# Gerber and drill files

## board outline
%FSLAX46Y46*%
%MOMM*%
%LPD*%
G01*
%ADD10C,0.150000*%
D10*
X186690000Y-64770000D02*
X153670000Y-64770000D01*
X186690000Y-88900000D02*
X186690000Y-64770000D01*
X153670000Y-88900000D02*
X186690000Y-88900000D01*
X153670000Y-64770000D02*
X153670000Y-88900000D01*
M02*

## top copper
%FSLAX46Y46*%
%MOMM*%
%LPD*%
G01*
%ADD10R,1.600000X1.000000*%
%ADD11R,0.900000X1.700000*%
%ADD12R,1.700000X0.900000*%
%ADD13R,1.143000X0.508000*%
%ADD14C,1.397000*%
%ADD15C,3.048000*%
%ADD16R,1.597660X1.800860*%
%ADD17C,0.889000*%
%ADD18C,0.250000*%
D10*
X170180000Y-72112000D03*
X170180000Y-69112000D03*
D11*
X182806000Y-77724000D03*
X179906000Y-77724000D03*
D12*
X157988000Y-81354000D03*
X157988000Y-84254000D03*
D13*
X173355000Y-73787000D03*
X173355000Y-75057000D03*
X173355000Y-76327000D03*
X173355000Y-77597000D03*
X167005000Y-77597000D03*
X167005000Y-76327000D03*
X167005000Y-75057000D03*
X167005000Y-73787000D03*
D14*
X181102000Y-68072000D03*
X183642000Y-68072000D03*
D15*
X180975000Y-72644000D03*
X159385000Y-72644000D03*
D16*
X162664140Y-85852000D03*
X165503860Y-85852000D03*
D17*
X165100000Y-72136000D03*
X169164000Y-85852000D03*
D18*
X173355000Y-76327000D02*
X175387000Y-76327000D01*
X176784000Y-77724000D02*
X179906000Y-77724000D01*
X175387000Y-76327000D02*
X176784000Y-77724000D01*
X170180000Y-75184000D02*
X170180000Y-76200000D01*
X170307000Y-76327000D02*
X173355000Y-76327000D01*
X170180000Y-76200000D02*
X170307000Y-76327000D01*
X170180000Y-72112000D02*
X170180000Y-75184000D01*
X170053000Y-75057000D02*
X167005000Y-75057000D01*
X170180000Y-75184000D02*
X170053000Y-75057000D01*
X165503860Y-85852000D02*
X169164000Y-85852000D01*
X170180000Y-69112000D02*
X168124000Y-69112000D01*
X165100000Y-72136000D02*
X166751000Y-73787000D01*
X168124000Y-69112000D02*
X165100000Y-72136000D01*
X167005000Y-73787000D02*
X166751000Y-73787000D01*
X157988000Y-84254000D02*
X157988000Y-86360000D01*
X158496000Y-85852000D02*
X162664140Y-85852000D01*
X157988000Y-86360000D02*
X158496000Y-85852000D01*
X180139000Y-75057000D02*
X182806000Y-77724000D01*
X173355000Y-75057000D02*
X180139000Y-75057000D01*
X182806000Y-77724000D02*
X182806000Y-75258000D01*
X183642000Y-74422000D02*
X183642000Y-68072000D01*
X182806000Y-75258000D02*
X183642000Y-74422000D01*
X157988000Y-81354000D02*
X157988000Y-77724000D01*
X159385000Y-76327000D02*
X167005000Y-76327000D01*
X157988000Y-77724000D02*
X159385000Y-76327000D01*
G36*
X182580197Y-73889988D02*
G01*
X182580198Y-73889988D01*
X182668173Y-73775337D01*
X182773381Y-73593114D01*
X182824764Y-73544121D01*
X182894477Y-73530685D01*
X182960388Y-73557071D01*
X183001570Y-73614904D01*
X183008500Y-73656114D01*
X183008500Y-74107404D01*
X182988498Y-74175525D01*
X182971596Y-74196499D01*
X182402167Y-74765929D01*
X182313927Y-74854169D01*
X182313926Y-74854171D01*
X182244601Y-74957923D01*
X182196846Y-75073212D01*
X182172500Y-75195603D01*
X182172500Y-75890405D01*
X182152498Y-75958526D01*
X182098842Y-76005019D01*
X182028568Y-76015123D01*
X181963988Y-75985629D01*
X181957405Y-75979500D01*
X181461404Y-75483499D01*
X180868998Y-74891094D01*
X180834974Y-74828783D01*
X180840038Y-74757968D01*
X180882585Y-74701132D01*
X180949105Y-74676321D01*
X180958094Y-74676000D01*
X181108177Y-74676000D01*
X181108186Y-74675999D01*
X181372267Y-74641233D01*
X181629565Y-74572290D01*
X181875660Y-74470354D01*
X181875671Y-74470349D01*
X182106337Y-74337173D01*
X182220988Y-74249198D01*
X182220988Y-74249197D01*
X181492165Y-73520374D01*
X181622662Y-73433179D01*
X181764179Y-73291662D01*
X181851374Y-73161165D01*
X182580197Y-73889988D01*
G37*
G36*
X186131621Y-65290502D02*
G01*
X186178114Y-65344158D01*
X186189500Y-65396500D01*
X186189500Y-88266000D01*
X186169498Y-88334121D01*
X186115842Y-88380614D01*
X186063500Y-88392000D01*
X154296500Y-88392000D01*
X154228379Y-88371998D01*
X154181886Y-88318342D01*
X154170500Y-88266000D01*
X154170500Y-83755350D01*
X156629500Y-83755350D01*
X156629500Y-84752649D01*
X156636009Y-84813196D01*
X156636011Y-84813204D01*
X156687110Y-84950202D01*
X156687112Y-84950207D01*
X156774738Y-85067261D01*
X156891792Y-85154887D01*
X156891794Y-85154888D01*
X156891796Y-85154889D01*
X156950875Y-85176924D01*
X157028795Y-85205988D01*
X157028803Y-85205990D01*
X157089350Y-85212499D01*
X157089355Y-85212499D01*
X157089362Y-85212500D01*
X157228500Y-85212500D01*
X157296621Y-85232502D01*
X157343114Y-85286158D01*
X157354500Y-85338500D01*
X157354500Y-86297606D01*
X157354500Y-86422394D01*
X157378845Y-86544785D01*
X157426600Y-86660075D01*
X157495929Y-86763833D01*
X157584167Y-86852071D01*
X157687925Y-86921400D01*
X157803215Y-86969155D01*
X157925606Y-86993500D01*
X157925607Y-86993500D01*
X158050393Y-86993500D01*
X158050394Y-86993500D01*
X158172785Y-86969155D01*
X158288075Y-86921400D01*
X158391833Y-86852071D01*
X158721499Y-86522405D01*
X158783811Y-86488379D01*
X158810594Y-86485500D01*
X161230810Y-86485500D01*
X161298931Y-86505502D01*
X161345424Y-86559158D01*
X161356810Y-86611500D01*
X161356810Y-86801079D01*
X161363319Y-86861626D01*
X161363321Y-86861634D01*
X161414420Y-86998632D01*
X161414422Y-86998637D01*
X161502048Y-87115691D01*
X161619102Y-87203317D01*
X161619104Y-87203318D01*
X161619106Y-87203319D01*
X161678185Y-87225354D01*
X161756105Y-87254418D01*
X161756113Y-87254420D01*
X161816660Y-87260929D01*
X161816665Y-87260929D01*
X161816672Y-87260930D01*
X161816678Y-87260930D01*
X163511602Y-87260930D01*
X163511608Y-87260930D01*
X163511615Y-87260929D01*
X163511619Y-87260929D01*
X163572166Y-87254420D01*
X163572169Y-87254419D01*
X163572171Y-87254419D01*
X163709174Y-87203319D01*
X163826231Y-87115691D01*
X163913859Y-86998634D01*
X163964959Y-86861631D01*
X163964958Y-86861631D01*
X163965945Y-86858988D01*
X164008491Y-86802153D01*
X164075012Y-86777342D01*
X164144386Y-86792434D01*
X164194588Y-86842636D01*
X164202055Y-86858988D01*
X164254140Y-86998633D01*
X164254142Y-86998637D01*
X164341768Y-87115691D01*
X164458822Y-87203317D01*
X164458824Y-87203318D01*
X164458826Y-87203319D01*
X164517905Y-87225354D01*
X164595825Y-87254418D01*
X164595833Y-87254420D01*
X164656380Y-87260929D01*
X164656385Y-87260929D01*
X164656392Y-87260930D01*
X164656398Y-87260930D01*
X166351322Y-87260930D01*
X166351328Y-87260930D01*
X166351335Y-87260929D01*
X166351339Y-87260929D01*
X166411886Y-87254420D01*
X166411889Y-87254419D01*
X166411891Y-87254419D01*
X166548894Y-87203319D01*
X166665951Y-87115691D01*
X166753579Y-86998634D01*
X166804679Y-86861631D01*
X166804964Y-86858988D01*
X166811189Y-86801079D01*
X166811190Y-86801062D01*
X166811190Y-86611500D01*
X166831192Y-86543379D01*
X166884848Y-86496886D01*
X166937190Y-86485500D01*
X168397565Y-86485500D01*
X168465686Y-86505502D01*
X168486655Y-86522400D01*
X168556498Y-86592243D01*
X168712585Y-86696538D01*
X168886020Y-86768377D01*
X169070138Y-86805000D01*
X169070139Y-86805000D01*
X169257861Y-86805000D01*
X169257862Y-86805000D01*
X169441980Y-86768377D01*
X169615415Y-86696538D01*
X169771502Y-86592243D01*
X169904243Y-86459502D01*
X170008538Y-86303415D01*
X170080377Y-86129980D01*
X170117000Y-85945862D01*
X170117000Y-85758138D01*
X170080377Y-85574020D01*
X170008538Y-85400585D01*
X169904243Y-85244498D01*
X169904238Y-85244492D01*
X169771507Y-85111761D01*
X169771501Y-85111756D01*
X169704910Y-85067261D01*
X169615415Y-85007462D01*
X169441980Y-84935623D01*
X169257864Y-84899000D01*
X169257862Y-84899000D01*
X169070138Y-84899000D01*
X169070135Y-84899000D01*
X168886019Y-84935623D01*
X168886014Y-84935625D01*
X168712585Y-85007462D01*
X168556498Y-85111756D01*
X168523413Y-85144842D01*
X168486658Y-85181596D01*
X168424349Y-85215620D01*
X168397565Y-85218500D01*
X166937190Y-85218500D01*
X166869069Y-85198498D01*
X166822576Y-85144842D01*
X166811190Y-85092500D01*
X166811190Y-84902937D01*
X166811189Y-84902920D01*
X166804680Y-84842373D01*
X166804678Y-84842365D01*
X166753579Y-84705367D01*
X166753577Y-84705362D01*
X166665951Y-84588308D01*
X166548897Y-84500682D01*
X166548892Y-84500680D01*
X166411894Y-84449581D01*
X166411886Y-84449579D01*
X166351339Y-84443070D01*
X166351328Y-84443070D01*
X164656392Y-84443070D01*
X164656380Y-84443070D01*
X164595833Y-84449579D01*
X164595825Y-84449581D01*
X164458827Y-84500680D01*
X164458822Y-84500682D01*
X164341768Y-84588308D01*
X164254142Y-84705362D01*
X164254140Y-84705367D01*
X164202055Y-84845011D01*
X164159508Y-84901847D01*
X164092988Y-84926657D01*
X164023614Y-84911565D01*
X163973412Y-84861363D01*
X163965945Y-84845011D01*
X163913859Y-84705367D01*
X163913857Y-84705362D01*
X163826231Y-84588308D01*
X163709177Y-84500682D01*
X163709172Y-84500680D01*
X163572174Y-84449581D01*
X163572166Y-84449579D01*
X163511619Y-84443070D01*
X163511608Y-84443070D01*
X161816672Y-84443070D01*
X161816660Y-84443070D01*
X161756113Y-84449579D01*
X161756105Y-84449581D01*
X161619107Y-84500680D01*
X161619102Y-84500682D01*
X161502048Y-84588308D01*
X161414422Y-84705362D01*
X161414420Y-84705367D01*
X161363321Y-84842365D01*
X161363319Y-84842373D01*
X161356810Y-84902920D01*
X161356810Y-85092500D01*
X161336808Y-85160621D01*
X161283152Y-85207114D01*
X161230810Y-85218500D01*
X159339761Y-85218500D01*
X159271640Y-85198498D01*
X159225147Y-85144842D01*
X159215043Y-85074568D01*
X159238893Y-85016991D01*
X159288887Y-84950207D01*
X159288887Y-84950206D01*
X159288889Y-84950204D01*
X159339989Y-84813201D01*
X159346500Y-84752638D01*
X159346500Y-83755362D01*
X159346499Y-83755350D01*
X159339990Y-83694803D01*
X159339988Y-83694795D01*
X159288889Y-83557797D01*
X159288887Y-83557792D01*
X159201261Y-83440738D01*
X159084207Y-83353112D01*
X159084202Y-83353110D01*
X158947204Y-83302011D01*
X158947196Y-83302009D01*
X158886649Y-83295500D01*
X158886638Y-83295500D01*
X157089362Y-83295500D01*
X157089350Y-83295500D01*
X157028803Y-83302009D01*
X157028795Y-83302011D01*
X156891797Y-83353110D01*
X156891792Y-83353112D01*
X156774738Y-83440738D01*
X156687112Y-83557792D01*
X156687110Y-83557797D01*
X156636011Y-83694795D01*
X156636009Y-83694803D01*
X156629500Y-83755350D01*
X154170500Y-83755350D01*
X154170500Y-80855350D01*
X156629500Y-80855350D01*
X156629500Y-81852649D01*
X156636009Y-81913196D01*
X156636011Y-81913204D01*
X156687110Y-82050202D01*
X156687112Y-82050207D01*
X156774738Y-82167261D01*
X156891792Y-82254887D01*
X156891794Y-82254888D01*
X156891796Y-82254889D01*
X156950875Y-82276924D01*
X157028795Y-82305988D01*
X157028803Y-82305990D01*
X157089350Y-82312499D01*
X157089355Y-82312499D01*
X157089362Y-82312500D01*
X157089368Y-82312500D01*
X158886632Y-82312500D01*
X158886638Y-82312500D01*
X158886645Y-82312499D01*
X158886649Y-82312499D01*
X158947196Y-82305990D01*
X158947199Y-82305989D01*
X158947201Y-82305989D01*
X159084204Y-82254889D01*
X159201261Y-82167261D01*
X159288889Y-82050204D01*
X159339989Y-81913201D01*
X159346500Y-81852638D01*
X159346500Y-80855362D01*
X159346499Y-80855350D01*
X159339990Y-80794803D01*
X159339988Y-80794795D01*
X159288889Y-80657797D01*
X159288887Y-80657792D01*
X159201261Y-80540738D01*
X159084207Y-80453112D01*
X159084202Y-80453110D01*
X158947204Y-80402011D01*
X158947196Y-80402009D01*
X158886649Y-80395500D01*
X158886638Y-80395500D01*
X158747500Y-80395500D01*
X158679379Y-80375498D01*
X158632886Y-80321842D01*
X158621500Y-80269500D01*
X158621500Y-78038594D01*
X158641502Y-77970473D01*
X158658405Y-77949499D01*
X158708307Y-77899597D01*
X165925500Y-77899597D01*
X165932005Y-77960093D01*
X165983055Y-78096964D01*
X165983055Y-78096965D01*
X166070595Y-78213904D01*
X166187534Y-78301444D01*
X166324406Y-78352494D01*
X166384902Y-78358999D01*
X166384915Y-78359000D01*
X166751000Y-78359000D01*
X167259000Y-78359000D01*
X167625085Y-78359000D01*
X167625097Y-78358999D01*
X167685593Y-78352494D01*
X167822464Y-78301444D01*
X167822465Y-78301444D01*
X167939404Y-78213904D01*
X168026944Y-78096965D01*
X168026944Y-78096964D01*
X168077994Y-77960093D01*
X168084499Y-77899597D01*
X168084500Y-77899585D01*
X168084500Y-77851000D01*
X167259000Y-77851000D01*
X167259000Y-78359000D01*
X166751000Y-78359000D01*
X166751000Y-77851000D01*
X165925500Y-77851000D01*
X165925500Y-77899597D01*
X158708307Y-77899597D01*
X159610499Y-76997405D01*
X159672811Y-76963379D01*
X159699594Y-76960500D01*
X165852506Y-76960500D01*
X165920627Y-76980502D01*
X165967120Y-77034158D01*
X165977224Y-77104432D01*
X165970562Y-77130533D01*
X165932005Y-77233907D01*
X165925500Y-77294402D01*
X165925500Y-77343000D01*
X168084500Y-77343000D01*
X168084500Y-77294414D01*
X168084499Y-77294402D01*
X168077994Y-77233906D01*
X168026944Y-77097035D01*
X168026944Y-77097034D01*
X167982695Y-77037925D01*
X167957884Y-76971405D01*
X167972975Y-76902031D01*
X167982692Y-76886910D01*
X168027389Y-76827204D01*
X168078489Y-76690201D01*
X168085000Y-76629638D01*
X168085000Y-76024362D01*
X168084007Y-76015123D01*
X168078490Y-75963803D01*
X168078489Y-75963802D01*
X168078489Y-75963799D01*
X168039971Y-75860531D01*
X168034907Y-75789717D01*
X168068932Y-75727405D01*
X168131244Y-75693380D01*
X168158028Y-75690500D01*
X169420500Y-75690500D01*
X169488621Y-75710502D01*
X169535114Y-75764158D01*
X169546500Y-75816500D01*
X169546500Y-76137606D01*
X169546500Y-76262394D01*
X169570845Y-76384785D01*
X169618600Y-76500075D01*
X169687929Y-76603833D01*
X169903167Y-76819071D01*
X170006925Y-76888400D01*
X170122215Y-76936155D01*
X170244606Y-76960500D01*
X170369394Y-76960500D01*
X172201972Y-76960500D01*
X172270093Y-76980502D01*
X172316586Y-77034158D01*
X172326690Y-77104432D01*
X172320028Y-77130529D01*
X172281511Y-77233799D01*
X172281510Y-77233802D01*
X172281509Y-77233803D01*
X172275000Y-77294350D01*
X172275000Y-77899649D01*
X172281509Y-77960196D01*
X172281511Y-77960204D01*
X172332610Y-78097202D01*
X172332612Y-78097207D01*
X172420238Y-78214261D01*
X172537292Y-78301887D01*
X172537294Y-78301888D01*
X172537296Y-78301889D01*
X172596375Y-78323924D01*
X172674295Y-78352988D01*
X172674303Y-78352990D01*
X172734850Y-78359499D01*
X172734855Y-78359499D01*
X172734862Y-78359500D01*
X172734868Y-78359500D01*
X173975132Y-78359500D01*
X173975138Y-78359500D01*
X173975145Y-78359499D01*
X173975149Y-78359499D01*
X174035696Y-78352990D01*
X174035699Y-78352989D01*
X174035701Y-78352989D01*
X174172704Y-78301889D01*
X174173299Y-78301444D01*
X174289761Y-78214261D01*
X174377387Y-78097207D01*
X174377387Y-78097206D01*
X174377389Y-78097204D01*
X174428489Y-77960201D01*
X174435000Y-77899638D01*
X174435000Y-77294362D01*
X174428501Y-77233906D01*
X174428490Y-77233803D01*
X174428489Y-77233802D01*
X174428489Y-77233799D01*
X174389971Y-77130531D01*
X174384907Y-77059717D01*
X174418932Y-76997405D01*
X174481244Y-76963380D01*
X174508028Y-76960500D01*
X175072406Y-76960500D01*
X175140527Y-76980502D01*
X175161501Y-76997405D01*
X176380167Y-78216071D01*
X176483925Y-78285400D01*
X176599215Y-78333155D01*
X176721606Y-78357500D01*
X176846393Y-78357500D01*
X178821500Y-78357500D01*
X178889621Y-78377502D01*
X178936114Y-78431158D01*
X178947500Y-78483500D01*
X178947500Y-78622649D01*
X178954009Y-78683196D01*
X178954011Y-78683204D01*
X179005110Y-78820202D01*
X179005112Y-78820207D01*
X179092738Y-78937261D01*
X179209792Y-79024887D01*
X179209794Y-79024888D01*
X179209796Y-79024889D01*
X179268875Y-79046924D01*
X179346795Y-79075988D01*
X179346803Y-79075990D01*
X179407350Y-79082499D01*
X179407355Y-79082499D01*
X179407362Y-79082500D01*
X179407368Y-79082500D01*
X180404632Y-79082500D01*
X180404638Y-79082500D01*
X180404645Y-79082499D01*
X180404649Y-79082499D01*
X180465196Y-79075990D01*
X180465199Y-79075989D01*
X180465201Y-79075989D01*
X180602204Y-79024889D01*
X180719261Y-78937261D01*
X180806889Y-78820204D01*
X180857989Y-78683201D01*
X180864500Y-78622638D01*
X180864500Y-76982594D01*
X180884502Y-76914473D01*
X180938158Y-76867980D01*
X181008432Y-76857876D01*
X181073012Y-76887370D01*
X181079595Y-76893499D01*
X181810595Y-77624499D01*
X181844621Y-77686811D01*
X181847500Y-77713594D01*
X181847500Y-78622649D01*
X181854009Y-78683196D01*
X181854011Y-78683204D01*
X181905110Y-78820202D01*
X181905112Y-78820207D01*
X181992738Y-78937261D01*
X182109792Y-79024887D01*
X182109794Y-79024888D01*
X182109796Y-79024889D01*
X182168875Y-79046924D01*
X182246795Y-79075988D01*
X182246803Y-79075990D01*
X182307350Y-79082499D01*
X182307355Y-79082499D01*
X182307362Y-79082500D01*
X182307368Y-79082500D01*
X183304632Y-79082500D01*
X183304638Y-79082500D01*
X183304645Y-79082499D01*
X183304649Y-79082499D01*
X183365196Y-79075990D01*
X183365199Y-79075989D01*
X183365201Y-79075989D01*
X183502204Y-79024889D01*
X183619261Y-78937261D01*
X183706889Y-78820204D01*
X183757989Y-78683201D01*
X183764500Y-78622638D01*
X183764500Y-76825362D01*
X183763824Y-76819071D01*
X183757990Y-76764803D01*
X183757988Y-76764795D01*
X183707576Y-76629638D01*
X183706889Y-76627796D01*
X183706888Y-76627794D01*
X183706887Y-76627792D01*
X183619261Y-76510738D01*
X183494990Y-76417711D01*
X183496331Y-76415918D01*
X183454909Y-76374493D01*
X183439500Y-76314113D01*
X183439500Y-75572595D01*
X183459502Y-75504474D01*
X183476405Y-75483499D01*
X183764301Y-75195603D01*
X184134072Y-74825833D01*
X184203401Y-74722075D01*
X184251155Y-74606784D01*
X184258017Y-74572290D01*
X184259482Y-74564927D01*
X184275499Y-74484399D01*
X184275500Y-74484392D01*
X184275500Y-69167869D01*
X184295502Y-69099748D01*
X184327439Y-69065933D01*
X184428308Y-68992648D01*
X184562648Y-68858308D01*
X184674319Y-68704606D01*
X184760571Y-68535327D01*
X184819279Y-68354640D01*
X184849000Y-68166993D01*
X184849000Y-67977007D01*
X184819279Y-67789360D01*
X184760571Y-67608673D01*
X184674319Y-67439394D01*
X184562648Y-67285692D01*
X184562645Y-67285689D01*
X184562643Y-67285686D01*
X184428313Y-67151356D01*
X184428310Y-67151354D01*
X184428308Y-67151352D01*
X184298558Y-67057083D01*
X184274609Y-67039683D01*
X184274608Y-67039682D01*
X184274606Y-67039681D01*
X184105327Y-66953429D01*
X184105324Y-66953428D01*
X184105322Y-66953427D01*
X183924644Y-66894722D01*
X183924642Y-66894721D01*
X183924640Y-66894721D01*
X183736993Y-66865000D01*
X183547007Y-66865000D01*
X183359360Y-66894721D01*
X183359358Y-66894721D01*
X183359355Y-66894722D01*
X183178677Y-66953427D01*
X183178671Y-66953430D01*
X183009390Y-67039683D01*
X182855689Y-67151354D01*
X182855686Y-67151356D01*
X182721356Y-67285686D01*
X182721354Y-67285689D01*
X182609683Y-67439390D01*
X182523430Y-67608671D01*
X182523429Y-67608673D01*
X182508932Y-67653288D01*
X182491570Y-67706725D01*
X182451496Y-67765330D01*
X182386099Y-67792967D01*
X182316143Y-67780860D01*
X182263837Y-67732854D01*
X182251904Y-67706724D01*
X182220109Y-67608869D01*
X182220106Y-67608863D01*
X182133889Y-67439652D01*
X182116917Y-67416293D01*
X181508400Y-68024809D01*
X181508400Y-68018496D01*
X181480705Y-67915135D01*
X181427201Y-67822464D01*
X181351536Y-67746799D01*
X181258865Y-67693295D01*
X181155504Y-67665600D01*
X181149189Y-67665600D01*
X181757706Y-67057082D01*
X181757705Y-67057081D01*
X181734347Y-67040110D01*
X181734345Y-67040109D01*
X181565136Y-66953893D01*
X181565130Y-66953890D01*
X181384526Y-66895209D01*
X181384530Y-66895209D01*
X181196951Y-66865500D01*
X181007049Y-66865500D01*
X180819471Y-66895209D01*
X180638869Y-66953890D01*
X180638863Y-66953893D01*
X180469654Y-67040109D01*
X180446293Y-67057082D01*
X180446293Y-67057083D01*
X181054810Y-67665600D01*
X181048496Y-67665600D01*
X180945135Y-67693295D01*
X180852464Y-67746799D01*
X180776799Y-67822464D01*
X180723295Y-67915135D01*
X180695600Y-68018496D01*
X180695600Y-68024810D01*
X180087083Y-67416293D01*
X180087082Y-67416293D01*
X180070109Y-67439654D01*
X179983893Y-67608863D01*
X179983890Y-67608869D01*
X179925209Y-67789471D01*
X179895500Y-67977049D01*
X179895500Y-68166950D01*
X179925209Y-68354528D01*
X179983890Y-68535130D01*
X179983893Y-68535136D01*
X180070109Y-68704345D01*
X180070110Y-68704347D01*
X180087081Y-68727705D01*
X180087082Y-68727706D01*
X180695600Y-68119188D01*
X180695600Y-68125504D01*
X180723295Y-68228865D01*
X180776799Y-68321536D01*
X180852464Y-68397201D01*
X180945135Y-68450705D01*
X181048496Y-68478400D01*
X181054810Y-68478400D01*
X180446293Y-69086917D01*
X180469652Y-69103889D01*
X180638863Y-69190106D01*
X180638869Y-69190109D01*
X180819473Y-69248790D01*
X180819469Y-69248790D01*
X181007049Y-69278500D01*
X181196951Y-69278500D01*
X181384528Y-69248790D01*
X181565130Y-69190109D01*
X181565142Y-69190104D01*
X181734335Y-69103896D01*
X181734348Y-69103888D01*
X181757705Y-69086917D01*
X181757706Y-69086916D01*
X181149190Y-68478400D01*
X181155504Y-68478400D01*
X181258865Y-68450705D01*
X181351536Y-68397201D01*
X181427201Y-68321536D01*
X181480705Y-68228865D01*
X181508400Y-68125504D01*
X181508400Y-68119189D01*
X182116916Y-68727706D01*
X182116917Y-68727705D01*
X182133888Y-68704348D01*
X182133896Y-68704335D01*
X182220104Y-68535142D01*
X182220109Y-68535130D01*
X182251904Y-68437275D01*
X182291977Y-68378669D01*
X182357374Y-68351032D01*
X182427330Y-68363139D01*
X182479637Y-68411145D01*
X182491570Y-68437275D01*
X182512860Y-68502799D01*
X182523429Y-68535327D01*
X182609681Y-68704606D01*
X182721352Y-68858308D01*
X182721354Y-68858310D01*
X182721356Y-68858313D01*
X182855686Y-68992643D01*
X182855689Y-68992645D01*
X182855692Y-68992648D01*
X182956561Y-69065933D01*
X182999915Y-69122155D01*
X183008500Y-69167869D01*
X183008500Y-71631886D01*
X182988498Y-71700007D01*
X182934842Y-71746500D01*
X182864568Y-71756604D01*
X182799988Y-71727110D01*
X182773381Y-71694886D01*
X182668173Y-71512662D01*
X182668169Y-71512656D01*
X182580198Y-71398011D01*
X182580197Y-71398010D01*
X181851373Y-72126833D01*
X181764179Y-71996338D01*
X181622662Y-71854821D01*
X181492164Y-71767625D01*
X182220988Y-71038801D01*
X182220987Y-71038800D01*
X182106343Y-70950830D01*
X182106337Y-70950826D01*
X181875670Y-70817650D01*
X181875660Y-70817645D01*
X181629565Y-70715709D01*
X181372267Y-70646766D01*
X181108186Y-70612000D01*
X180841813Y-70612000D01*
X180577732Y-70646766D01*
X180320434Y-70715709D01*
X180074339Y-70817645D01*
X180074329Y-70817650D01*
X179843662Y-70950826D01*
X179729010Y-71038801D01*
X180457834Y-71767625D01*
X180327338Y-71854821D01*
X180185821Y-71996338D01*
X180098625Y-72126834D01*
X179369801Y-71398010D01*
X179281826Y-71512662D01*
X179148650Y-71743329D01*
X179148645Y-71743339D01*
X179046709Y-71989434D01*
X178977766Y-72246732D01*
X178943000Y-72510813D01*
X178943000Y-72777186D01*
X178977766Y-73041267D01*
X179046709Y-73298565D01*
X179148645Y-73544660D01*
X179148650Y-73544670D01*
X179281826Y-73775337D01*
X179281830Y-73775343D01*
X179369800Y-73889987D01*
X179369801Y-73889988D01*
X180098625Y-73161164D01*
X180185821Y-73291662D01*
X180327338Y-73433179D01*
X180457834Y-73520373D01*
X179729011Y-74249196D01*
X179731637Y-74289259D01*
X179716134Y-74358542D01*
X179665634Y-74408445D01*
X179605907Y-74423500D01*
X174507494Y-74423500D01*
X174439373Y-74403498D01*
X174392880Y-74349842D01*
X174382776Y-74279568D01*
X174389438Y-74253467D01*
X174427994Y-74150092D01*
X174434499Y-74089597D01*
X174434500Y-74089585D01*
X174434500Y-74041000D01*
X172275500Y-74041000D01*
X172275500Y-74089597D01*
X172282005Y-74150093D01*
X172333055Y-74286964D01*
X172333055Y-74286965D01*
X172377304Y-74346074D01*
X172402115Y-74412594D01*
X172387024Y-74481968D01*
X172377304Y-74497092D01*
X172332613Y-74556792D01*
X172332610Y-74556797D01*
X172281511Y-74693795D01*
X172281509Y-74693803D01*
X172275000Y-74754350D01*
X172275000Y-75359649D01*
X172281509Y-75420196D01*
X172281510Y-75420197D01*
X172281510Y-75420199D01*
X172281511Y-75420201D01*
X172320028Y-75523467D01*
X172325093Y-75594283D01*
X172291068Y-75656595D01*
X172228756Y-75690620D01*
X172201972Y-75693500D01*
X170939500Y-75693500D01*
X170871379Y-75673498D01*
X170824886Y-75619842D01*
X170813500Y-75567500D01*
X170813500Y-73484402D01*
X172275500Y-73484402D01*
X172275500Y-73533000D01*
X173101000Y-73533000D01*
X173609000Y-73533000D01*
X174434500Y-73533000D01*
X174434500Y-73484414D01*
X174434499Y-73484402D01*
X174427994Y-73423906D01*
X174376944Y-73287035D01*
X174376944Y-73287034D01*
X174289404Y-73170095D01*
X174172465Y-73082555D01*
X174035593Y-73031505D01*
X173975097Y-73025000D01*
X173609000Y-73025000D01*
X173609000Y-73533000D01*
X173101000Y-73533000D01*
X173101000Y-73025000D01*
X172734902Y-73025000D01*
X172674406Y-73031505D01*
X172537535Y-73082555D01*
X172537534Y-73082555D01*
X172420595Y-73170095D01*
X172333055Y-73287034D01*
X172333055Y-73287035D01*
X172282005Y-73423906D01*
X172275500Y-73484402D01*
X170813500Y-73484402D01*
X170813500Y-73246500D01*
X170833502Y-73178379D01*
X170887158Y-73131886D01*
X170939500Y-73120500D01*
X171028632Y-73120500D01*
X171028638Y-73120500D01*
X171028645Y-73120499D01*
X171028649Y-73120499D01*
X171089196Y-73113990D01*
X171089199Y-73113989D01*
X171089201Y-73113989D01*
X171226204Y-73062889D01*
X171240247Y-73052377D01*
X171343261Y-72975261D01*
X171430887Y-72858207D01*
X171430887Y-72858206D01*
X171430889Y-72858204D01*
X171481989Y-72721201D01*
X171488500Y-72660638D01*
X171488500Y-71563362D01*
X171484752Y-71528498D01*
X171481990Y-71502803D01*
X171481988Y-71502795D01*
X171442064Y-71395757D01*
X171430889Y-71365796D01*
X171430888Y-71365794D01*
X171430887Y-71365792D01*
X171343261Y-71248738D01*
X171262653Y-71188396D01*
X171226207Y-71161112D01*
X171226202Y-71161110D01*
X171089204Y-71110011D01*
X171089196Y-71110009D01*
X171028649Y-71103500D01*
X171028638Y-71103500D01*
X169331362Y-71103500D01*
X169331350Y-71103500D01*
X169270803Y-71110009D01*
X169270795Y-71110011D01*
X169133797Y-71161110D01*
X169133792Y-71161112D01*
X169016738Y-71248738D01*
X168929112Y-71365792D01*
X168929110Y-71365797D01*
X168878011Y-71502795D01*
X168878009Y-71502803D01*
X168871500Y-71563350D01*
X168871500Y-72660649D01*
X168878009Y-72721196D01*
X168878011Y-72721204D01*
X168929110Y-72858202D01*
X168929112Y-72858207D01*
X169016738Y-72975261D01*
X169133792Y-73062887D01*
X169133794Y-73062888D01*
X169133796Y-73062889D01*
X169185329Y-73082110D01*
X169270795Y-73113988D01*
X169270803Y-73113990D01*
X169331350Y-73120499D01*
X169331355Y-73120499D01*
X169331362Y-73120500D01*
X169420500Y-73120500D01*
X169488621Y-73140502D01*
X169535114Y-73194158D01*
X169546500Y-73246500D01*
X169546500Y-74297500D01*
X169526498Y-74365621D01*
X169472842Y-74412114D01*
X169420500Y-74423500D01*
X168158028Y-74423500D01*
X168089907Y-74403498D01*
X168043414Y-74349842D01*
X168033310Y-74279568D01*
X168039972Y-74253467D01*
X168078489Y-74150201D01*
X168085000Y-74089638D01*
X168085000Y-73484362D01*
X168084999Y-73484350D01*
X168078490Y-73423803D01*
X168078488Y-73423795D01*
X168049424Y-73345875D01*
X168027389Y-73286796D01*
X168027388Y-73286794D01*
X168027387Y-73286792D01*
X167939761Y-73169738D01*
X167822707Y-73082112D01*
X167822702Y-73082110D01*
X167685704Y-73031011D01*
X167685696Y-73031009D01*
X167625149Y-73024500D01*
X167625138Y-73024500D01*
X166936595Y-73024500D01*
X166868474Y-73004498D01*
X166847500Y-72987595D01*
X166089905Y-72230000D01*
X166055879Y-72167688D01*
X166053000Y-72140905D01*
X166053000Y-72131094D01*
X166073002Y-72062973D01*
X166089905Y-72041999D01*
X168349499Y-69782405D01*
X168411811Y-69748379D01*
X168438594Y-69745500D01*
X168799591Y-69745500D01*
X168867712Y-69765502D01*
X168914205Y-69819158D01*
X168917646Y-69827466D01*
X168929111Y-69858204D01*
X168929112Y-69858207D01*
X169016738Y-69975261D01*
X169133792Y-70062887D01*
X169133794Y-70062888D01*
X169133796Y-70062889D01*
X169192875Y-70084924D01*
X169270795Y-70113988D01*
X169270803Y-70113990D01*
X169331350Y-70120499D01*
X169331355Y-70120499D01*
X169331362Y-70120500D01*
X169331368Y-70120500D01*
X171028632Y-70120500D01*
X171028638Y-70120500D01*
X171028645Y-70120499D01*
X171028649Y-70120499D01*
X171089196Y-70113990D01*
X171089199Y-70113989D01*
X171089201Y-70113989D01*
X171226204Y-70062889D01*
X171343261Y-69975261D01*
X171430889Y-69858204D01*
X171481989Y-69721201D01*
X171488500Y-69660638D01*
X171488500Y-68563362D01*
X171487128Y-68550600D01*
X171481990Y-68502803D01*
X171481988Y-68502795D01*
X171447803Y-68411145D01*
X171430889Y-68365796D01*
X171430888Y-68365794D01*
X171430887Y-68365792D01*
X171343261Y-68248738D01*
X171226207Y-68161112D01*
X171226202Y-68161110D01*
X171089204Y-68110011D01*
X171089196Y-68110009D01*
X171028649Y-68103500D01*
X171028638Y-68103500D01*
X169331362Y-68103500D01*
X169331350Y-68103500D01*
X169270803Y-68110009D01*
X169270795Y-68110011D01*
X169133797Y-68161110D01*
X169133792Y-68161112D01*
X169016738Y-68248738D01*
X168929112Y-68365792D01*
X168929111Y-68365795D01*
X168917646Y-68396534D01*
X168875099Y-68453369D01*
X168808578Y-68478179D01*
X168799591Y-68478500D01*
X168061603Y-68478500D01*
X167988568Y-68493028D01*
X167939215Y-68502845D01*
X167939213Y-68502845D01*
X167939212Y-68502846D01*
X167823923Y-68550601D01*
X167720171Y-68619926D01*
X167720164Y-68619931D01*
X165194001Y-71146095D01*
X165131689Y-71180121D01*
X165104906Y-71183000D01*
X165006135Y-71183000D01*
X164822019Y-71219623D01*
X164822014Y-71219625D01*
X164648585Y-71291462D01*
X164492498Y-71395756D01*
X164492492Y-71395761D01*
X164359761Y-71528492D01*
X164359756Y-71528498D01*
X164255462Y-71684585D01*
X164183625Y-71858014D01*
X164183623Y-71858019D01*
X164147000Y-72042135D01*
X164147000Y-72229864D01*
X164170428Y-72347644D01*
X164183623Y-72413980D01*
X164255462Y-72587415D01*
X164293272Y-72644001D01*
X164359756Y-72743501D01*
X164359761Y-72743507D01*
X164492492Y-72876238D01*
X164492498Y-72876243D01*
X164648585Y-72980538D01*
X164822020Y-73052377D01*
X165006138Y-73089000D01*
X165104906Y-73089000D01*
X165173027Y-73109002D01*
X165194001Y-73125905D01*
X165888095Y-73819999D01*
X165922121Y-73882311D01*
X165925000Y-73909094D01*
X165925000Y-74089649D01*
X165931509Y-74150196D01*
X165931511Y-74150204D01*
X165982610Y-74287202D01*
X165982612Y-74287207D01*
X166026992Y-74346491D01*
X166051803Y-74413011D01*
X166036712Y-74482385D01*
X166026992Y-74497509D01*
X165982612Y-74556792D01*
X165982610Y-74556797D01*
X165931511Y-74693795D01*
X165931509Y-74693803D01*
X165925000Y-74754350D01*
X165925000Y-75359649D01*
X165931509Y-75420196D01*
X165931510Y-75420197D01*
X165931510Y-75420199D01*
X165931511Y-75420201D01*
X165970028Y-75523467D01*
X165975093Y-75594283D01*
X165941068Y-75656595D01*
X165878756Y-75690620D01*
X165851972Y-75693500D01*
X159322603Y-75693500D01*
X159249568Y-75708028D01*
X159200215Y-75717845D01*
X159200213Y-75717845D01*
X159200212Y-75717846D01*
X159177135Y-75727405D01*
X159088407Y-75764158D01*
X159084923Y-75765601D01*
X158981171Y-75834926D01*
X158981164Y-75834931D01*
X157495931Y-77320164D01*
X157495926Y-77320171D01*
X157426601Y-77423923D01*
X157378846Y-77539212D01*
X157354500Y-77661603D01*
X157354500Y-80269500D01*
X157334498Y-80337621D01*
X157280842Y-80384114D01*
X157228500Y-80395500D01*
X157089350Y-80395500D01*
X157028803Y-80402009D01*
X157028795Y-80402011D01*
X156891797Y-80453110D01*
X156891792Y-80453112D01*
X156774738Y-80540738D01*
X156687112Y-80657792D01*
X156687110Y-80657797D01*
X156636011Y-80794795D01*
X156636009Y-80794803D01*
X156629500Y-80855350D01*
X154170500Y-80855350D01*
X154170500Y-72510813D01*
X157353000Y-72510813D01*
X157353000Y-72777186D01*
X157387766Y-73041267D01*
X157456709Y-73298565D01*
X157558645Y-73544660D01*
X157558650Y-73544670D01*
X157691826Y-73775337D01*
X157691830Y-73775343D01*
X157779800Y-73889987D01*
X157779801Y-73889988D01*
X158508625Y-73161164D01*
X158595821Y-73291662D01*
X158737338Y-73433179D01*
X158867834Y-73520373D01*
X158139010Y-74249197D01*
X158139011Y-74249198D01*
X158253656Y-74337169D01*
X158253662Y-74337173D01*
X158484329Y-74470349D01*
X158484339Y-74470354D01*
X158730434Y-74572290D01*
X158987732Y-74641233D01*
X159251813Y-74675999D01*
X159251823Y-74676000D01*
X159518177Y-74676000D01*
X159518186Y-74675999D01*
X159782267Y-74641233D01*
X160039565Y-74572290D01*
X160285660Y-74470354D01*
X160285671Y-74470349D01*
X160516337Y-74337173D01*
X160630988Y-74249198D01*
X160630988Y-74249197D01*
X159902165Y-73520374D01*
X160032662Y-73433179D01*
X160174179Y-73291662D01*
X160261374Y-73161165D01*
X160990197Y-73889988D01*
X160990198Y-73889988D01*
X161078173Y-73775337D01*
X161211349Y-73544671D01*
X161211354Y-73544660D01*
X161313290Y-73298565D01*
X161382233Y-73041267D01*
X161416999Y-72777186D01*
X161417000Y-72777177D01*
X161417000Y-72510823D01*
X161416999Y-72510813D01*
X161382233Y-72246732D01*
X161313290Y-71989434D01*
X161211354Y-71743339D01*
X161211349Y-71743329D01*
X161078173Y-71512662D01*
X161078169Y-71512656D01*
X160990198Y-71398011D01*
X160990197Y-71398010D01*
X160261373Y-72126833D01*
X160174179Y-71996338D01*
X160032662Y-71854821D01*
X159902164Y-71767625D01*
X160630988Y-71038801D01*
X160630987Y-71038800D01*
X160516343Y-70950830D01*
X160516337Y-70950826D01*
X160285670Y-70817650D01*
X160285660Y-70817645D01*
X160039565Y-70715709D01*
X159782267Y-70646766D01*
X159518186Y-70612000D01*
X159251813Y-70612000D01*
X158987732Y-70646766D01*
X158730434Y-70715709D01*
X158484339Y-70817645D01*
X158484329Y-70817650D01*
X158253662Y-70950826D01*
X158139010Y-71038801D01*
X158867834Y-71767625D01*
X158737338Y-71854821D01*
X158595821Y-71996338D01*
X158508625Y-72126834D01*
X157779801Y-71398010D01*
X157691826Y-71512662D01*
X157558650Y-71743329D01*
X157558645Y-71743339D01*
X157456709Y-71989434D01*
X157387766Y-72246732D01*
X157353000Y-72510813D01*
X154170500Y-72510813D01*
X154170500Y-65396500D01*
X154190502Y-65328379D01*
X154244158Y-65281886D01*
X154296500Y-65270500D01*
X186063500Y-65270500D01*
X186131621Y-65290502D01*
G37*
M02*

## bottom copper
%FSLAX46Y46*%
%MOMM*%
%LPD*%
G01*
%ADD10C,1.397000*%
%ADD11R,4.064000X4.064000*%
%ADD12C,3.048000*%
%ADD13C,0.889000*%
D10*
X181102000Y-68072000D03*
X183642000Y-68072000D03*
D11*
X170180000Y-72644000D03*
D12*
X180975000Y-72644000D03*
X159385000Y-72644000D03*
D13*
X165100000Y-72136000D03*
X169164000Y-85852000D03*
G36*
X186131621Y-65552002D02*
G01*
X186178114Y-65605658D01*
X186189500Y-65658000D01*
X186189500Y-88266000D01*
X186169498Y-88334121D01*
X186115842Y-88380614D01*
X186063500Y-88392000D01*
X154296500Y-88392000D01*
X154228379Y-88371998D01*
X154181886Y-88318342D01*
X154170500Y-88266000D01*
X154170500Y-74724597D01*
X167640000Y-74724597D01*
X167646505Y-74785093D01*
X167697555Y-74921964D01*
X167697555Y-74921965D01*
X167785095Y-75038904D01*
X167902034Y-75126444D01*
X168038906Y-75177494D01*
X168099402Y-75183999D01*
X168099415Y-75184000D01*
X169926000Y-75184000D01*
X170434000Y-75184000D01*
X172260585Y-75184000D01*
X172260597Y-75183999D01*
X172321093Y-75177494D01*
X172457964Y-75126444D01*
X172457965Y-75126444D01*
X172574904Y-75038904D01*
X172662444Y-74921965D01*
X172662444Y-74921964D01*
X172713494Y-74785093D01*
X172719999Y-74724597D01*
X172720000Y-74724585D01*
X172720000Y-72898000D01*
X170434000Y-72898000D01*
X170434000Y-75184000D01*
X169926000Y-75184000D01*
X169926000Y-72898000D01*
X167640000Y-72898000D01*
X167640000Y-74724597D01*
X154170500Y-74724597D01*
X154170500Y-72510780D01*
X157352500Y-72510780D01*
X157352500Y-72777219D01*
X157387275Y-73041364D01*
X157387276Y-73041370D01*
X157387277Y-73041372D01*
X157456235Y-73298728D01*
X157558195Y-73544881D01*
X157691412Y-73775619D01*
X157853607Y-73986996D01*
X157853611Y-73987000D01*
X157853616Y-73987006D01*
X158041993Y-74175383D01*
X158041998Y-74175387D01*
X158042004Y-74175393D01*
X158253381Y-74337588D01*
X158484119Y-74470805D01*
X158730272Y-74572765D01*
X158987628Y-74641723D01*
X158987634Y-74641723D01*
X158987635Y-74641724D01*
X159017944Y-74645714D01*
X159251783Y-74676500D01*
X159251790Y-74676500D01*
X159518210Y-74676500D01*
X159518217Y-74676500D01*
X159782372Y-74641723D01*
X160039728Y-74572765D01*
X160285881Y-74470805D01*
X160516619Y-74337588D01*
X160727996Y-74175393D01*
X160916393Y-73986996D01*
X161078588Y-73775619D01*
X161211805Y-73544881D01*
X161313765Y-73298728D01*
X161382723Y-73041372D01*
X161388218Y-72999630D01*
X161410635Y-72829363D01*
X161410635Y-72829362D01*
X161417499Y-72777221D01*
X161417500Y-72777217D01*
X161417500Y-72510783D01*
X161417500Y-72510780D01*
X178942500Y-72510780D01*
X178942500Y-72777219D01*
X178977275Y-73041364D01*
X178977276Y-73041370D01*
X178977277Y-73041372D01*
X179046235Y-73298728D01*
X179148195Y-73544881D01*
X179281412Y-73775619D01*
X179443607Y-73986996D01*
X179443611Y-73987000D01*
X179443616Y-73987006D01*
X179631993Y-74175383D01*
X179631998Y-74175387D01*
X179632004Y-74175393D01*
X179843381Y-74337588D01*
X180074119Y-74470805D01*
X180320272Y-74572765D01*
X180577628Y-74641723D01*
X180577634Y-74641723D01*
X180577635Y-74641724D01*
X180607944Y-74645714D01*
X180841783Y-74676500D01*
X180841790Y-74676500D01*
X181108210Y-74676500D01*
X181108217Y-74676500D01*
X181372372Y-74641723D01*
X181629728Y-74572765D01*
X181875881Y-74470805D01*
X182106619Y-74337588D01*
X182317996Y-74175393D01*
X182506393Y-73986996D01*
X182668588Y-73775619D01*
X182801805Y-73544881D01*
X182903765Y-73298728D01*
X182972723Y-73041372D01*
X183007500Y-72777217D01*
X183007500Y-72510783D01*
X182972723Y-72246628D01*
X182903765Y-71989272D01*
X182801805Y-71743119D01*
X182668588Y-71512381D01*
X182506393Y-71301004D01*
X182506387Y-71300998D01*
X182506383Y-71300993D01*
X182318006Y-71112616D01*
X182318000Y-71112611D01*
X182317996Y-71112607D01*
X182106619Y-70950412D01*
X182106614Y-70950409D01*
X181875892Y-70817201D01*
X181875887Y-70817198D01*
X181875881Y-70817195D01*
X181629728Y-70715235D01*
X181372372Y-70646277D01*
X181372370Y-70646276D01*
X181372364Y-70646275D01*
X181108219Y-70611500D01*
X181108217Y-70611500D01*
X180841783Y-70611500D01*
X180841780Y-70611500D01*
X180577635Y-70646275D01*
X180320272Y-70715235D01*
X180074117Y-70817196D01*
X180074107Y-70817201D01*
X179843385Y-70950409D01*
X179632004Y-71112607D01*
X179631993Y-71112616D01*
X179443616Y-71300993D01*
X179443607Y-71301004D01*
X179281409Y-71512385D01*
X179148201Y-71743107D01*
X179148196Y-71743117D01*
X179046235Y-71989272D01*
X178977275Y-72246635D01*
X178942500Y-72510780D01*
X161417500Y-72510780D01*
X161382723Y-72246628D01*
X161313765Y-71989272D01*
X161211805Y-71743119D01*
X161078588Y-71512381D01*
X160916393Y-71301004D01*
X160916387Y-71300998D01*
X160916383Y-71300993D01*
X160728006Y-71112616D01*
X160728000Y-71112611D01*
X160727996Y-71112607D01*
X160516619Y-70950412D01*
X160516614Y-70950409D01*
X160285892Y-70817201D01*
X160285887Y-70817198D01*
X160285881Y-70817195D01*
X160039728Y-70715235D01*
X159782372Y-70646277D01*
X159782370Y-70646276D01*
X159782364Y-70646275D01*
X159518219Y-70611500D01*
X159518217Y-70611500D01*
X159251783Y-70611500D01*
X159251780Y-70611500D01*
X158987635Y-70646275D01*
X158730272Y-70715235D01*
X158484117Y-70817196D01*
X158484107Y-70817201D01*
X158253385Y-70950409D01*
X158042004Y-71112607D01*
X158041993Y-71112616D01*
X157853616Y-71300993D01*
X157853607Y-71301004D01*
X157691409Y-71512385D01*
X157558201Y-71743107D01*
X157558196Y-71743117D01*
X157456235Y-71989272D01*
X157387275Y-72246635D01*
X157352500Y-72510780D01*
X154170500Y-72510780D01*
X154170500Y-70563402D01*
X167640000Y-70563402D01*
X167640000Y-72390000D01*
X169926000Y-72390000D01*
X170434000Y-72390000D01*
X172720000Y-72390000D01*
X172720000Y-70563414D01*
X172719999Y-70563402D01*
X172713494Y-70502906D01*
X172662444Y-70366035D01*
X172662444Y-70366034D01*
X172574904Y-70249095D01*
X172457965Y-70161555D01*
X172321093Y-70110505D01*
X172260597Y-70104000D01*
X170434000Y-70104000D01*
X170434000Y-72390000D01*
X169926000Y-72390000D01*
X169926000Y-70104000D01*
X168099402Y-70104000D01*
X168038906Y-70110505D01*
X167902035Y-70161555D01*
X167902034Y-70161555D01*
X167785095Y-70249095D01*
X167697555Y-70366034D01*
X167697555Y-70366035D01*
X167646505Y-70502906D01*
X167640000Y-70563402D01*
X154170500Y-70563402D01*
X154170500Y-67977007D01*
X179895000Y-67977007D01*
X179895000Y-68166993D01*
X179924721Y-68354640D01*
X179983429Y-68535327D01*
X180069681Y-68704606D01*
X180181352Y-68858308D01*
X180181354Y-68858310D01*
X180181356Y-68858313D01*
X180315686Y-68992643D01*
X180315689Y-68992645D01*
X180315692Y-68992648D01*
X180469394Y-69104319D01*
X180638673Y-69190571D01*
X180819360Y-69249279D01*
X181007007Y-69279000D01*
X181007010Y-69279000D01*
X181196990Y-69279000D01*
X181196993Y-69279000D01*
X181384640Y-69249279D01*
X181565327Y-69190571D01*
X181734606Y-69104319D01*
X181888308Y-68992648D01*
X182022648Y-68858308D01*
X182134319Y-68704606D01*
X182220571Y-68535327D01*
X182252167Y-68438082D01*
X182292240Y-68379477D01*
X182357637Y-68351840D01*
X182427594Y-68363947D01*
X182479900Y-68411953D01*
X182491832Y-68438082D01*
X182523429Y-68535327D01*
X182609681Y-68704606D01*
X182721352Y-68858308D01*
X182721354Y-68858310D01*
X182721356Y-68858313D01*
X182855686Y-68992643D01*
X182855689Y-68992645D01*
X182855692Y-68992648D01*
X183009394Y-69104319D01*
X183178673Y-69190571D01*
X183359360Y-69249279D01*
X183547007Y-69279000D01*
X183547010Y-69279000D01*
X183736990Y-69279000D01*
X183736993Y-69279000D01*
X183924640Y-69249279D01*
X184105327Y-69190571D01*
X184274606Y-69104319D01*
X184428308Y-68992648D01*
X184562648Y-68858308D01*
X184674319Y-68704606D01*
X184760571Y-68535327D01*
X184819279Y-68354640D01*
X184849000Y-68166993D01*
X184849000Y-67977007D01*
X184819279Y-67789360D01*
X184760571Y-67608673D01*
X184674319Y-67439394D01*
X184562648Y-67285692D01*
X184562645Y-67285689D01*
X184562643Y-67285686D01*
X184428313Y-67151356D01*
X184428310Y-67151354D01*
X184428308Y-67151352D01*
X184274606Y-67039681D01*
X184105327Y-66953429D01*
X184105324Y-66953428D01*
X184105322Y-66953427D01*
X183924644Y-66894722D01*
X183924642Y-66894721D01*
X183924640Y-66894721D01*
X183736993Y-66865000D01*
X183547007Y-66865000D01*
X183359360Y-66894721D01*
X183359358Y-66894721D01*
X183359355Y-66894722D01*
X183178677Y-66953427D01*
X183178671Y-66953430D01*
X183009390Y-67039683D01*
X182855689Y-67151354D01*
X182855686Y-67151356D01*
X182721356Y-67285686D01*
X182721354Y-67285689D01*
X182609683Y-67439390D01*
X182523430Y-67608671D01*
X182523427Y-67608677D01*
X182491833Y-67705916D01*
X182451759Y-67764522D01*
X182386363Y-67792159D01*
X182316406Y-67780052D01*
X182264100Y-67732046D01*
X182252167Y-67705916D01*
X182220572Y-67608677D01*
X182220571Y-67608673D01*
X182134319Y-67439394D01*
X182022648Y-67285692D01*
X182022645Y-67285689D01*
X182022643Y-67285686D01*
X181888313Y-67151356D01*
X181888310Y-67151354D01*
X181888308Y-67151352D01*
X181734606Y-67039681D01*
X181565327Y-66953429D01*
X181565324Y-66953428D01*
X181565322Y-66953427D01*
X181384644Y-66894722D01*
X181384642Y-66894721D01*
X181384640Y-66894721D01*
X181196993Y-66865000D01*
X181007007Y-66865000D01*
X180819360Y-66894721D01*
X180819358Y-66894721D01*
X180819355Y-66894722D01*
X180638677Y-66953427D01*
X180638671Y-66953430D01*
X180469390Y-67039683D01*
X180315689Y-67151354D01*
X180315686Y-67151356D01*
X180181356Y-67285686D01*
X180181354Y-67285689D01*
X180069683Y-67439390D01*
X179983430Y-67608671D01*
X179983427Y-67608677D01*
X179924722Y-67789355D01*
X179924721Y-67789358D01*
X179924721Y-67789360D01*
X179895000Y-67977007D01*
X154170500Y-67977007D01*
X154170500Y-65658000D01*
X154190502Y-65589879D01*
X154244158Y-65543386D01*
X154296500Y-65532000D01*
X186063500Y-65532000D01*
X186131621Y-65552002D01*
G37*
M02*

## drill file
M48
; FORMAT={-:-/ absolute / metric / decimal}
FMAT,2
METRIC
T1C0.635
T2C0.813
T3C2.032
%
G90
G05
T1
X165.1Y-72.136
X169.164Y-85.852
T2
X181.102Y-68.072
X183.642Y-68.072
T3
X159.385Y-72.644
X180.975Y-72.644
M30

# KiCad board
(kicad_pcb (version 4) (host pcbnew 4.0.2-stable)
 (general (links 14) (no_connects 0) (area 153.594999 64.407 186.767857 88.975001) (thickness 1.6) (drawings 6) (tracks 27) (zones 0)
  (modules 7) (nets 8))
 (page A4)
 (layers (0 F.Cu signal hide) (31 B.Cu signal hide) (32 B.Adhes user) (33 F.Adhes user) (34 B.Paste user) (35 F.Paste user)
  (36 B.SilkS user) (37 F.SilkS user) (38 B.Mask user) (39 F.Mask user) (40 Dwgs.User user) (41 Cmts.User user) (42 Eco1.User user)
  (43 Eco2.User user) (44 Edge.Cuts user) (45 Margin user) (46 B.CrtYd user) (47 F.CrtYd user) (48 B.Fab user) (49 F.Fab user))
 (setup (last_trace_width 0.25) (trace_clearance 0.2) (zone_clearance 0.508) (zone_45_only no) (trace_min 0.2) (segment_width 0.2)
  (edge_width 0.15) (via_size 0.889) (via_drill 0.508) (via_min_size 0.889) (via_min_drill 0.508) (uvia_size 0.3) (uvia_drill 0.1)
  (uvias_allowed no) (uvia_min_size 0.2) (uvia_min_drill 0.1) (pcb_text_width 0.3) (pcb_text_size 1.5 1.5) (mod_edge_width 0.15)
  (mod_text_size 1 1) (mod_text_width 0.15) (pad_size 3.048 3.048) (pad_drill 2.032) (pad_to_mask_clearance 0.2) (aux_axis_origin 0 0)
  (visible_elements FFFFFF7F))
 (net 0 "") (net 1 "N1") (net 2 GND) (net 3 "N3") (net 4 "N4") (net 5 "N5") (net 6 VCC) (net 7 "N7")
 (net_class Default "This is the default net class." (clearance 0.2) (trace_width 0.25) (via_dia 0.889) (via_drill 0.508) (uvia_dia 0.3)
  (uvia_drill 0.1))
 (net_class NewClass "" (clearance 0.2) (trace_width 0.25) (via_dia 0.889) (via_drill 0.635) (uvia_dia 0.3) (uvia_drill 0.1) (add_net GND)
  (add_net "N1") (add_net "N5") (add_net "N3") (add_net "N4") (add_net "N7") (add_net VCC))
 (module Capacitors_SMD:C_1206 (layer F.Cu) (at 170.18 70.612 90)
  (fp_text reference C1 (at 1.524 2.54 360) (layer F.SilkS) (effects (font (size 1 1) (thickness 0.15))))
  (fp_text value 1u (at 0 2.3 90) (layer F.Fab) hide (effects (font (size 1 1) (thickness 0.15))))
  (pad 1 smd rect (at -1.5 0 90) (size 1 1.6) (layers F.Cu F.Paste F.Mask) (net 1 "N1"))
  (pad 2 smd rect (at 1.5 0 90) (size 1 1.6) (layers F.Cu F.Paste F.Mask) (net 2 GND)))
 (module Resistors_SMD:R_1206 (layer F.Cu) (at 181.356 77.724 180)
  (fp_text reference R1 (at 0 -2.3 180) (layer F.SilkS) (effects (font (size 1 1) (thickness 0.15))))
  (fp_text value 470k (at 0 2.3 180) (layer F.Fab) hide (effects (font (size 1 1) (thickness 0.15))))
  (pad 1 smd rect (at -1.45 0 180) (size 0.9 1.7) (layers F.Cu F.Paste F.Mask) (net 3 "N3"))
  (pad 2 smd rect (at 1.45 0 180) (size 0.9 1.7) (layers F.Cu F.Paste F.Mask) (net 1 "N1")))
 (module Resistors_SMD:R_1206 (layer F.Cu) (at 157.988 82.804 270)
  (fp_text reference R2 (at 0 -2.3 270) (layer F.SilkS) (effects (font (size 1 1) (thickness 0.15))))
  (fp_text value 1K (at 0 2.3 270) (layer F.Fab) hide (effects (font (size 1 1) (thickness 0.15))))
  (pad 1 smd rect (at -1.45 0 270) (size 0.9 1.7) (layers F.Cu F.Paste F.Mask) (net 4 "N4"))
  (pad 2 smd rect (at 1.45 0 270) (size 0.9 1.7) (layers F.Cu F.Paste F.Mask) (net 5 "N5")))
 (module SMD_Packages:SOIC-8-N (layer F.Cu) (at 170.18 75.692 270)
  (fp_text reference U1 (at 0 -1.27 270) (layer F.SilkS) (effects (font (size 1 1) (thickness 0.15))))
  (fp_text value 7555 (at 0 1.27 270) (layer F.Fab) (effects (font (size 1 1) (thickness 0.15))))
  (pad 8 smd rect (at -1.905 -3.175 270) (size 0.508 1.143) (layers F.Cu F.Paste F.Mask) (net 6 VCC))
  (pad 7 smd rect (at -0.635 -3.175 270) (size 0.508 1.143) (layers F.Cu F.Paste F.Mask) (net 3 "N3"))
  (pad 6 smd rect (at 0.635 -3.175 270) (size 0.508 1.143) (layers F.Cu F.Paste F.Mask) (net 1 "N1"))
  (pad 5 smd rect (at 1.905 -3.175 270) (size 0.508 1.143) (layers F.Cu F.Paste F.Mask) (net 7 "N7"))
  (pad 4 smd rect (at 1.905 3.175 270) (size 0.508 1.143) (layers F.Cu F.Paste F.Mask) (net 6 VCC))
  (pad 3 smd rect (at 0.635 3.175 270) (size 0.508 1.143) (layers F.Cu F.Paste F.Mask) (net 4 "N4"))
  (pad 2 smd rect (at -0.635 3.175 270) (size 0.508 1.143) (layers F.Cu F.Paste F.Mask) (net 1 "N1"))
  (pad 1 smd rect (at -1.905 3.175 270) (size 0.508 1.143) (layers F.Cu F.Paste F.Mask) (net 2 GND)))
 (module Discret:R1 (layer F.Cu) (at 182.372 68.072)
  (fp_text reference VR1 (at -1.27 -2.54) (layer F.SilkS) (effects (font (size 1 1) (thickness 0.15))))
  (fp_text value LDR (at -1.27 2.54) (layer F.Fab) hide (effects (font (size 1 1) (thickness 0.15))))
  (pad 1 thru_hole circle (at -1.27 0) (size 1.397 1.397) (drill 0.8128) (layers *.Cu *.Mask F.SilkS) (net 6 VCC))
  (pad 2 thru_hole circle (at 1.27 0) (size 1.397 1.397) (drill 0.8128) (layers *.Cu *.Mask F.SilkS) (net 3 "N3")))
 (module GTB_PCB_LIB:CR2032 (layer B.Cu) (at 170.18 72.644 180)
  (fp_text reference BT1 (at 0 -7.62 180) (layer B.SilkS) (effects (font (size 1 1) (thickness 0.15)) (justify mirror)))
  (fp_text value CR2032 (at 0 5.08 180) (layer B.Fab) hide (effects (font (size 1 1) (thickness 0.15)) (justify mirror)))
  (pad 2 smd rect (at 0 0 180) (size 4.064 4.064) (layers B.Cu B.Paste B.Mask) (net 2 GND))
  (pad 1 thru_hole circle (at -10.795 0 180) (size 3.048 3.048) (drill 2.032) (layers *.Cu *.Mask B.SilkS) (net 6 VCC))
  (pad 1 thru_hole circle (at 10.795 0 180) (size 3.048 3.048) (drill 2.032) (layers *.Cu *.Mask B.SilkS) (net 6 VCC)))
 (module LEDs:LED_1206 (layer F.Cu) (at 164.084 85.852 180)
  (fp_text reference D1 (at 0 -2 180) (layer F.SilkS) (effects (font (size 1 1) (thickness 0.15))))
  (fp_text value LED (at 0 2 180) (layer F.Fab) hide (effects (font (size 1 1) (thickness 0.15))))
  (pad 2 smd rect (at 1.41986 0) (size 1.59766 1.80086) (layers F.Cu F.Paste F.Mask) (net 5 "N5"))
  (pad 1 smd rect (at -1.41986 0) (size 1.59766 1.80086) (layers F.Cu F.Paste F.Mask) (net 2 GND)))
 (gr_line (start 186.69 64.77) (end 153.67 64.77) (angle 90) (layer Edge.Cuts) (width 0.15))
 (gr_line (start 186.69 88.9) (end 186.69 64.77) (angle 90) (layer Edge.Cuts) (width 0.15))
 (gr_line (start 153.67 88.9) (end 186.69 88.9) (angle 90) (layer Edge.Cuts) (width 0.15))
 (gr_line (start 153.67 64.77) (end 153.67 88.9) (angle 90) (layer Edge.Cuts) (width 0.15))
 (segment (start 173.355 76.327) (end 175.387 76.327) (width 0.25) (layer F.Cu) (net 1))
 (segment (start 176.784 77.724) (end 179.906 77.724) (width 0.25) (layer F.Cu) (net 1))
 (segment (start 175.387 76.327) (end 176.784 77.724) (width 0.25) (layer F.Cu) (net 1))
 (segment (start 170.18 75.184) (end 170.18 76.2) (width 0.25) (layer F.Cu) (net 1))
 (segment (start 170.307 76.327) (end 173.355 76.327) (width 0.25) (layer F.Cu) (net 1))
 (segment (start 170.18 76.2) (end 170.307 76.327) (width 0.25) (layer F.Cu) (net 1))
 (segment (start 170.18 72.112) (end 170.18 75.184) (width 0.25) (layer F.Cu) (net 1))
 (segment (start 170.053 75.057) (end 167.005 75.057) (width 0.25) (layer F.Cu) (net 1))
 (segment (start 170.18 75.184) (end 170.053 75.057) (width 0.25) (layer F.Cu) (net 1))
 (via (at 165.1 72.136) (size 0.889) (drill 0.635) (layers F.Cu B.Cu) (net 2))
 (via (at 169.164 85.852) (size 0.889) (drill 0.635) (layers F.Cu B.Cu) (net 2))
 (segment (start 165.50386 85.852) (end 169.164 85.852) (width 0.25) (layer F.Cu) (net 2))
 (segment (start 170.18 69.112) (end 168.124 69.112) (width 0.25) (layer F.Cu) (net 2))
 (segment (start 165.1 72.136) (end 166.751 73.787) (width 0.25) (layer F.Cu) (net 2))
 (segment (start 168.124 69.112) (end 165.1 72.136) (width 0.25) (layer F.Cu) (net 2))
 (segment (start 167.005 73.787) (end 166.751 73.787) (width 0.25) (layer F.Cu) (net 2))
 (segment (start 157.988 84.254) (end 157.988 86.36) (width 0.25) (layer F.Cu) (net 5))
 (segment (start 158.496 85.852) (end 162.66414 85.852) (width 0.25) (layer F.Cu) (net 5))
 (segment (start 157.988 86.36) (end 158.496 85.852) (width 0.25) (layer F.Cu) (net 5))
 (segment (start 180.139 75.057) (end 182.806 77.724) (width 0.25) (layer F.Cu) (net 3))
 (segment (start 173.355 75.057) (end 180.139 75.057) (width 0.25) (layer F.Cu) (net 3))
 (segment (start 182.806 77.724) (end 182.806 75.258) (width 0.25) (layer F.Cu) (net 3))
 (segment (start 183.642 74.422) (end 183.642 68.072) (width 0.25) (layer F.Cu) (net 3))
 (segment (start 182.806 75.258) (end 183.642 74.422) (width 0.25) (layer F.Cu) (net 3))
 (segment (start 157.988 81.354) (end 157.988 77.724) (width 0.25) (layer F.Cu) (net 4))
 (segment (start 159.385 76.327) (end 167.005 76.327) (width 0.25) (layer F.Cu) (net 4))
 (segment (start 157.988 77.724) (end 159.385 76.327) (width 0.25) (layer F.Cu) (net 4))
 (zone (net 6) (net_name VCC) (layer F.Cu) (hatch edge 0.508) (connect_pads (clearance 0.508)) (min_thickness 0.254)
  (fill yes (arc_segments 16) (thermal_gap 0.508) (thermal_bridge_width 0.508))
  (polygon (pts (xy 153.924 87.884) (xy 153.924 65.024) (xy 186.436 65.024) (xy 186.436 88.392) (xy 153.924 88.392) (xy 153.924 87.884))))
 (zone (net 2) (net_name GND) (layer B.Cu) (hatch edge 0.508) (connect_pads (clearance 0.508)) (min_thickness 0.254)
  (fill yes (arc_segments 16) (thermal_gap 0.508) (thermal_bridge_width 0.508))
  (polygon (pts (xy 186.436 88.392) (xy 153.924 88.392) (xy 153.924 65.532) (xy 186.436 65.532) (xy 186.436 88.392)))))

